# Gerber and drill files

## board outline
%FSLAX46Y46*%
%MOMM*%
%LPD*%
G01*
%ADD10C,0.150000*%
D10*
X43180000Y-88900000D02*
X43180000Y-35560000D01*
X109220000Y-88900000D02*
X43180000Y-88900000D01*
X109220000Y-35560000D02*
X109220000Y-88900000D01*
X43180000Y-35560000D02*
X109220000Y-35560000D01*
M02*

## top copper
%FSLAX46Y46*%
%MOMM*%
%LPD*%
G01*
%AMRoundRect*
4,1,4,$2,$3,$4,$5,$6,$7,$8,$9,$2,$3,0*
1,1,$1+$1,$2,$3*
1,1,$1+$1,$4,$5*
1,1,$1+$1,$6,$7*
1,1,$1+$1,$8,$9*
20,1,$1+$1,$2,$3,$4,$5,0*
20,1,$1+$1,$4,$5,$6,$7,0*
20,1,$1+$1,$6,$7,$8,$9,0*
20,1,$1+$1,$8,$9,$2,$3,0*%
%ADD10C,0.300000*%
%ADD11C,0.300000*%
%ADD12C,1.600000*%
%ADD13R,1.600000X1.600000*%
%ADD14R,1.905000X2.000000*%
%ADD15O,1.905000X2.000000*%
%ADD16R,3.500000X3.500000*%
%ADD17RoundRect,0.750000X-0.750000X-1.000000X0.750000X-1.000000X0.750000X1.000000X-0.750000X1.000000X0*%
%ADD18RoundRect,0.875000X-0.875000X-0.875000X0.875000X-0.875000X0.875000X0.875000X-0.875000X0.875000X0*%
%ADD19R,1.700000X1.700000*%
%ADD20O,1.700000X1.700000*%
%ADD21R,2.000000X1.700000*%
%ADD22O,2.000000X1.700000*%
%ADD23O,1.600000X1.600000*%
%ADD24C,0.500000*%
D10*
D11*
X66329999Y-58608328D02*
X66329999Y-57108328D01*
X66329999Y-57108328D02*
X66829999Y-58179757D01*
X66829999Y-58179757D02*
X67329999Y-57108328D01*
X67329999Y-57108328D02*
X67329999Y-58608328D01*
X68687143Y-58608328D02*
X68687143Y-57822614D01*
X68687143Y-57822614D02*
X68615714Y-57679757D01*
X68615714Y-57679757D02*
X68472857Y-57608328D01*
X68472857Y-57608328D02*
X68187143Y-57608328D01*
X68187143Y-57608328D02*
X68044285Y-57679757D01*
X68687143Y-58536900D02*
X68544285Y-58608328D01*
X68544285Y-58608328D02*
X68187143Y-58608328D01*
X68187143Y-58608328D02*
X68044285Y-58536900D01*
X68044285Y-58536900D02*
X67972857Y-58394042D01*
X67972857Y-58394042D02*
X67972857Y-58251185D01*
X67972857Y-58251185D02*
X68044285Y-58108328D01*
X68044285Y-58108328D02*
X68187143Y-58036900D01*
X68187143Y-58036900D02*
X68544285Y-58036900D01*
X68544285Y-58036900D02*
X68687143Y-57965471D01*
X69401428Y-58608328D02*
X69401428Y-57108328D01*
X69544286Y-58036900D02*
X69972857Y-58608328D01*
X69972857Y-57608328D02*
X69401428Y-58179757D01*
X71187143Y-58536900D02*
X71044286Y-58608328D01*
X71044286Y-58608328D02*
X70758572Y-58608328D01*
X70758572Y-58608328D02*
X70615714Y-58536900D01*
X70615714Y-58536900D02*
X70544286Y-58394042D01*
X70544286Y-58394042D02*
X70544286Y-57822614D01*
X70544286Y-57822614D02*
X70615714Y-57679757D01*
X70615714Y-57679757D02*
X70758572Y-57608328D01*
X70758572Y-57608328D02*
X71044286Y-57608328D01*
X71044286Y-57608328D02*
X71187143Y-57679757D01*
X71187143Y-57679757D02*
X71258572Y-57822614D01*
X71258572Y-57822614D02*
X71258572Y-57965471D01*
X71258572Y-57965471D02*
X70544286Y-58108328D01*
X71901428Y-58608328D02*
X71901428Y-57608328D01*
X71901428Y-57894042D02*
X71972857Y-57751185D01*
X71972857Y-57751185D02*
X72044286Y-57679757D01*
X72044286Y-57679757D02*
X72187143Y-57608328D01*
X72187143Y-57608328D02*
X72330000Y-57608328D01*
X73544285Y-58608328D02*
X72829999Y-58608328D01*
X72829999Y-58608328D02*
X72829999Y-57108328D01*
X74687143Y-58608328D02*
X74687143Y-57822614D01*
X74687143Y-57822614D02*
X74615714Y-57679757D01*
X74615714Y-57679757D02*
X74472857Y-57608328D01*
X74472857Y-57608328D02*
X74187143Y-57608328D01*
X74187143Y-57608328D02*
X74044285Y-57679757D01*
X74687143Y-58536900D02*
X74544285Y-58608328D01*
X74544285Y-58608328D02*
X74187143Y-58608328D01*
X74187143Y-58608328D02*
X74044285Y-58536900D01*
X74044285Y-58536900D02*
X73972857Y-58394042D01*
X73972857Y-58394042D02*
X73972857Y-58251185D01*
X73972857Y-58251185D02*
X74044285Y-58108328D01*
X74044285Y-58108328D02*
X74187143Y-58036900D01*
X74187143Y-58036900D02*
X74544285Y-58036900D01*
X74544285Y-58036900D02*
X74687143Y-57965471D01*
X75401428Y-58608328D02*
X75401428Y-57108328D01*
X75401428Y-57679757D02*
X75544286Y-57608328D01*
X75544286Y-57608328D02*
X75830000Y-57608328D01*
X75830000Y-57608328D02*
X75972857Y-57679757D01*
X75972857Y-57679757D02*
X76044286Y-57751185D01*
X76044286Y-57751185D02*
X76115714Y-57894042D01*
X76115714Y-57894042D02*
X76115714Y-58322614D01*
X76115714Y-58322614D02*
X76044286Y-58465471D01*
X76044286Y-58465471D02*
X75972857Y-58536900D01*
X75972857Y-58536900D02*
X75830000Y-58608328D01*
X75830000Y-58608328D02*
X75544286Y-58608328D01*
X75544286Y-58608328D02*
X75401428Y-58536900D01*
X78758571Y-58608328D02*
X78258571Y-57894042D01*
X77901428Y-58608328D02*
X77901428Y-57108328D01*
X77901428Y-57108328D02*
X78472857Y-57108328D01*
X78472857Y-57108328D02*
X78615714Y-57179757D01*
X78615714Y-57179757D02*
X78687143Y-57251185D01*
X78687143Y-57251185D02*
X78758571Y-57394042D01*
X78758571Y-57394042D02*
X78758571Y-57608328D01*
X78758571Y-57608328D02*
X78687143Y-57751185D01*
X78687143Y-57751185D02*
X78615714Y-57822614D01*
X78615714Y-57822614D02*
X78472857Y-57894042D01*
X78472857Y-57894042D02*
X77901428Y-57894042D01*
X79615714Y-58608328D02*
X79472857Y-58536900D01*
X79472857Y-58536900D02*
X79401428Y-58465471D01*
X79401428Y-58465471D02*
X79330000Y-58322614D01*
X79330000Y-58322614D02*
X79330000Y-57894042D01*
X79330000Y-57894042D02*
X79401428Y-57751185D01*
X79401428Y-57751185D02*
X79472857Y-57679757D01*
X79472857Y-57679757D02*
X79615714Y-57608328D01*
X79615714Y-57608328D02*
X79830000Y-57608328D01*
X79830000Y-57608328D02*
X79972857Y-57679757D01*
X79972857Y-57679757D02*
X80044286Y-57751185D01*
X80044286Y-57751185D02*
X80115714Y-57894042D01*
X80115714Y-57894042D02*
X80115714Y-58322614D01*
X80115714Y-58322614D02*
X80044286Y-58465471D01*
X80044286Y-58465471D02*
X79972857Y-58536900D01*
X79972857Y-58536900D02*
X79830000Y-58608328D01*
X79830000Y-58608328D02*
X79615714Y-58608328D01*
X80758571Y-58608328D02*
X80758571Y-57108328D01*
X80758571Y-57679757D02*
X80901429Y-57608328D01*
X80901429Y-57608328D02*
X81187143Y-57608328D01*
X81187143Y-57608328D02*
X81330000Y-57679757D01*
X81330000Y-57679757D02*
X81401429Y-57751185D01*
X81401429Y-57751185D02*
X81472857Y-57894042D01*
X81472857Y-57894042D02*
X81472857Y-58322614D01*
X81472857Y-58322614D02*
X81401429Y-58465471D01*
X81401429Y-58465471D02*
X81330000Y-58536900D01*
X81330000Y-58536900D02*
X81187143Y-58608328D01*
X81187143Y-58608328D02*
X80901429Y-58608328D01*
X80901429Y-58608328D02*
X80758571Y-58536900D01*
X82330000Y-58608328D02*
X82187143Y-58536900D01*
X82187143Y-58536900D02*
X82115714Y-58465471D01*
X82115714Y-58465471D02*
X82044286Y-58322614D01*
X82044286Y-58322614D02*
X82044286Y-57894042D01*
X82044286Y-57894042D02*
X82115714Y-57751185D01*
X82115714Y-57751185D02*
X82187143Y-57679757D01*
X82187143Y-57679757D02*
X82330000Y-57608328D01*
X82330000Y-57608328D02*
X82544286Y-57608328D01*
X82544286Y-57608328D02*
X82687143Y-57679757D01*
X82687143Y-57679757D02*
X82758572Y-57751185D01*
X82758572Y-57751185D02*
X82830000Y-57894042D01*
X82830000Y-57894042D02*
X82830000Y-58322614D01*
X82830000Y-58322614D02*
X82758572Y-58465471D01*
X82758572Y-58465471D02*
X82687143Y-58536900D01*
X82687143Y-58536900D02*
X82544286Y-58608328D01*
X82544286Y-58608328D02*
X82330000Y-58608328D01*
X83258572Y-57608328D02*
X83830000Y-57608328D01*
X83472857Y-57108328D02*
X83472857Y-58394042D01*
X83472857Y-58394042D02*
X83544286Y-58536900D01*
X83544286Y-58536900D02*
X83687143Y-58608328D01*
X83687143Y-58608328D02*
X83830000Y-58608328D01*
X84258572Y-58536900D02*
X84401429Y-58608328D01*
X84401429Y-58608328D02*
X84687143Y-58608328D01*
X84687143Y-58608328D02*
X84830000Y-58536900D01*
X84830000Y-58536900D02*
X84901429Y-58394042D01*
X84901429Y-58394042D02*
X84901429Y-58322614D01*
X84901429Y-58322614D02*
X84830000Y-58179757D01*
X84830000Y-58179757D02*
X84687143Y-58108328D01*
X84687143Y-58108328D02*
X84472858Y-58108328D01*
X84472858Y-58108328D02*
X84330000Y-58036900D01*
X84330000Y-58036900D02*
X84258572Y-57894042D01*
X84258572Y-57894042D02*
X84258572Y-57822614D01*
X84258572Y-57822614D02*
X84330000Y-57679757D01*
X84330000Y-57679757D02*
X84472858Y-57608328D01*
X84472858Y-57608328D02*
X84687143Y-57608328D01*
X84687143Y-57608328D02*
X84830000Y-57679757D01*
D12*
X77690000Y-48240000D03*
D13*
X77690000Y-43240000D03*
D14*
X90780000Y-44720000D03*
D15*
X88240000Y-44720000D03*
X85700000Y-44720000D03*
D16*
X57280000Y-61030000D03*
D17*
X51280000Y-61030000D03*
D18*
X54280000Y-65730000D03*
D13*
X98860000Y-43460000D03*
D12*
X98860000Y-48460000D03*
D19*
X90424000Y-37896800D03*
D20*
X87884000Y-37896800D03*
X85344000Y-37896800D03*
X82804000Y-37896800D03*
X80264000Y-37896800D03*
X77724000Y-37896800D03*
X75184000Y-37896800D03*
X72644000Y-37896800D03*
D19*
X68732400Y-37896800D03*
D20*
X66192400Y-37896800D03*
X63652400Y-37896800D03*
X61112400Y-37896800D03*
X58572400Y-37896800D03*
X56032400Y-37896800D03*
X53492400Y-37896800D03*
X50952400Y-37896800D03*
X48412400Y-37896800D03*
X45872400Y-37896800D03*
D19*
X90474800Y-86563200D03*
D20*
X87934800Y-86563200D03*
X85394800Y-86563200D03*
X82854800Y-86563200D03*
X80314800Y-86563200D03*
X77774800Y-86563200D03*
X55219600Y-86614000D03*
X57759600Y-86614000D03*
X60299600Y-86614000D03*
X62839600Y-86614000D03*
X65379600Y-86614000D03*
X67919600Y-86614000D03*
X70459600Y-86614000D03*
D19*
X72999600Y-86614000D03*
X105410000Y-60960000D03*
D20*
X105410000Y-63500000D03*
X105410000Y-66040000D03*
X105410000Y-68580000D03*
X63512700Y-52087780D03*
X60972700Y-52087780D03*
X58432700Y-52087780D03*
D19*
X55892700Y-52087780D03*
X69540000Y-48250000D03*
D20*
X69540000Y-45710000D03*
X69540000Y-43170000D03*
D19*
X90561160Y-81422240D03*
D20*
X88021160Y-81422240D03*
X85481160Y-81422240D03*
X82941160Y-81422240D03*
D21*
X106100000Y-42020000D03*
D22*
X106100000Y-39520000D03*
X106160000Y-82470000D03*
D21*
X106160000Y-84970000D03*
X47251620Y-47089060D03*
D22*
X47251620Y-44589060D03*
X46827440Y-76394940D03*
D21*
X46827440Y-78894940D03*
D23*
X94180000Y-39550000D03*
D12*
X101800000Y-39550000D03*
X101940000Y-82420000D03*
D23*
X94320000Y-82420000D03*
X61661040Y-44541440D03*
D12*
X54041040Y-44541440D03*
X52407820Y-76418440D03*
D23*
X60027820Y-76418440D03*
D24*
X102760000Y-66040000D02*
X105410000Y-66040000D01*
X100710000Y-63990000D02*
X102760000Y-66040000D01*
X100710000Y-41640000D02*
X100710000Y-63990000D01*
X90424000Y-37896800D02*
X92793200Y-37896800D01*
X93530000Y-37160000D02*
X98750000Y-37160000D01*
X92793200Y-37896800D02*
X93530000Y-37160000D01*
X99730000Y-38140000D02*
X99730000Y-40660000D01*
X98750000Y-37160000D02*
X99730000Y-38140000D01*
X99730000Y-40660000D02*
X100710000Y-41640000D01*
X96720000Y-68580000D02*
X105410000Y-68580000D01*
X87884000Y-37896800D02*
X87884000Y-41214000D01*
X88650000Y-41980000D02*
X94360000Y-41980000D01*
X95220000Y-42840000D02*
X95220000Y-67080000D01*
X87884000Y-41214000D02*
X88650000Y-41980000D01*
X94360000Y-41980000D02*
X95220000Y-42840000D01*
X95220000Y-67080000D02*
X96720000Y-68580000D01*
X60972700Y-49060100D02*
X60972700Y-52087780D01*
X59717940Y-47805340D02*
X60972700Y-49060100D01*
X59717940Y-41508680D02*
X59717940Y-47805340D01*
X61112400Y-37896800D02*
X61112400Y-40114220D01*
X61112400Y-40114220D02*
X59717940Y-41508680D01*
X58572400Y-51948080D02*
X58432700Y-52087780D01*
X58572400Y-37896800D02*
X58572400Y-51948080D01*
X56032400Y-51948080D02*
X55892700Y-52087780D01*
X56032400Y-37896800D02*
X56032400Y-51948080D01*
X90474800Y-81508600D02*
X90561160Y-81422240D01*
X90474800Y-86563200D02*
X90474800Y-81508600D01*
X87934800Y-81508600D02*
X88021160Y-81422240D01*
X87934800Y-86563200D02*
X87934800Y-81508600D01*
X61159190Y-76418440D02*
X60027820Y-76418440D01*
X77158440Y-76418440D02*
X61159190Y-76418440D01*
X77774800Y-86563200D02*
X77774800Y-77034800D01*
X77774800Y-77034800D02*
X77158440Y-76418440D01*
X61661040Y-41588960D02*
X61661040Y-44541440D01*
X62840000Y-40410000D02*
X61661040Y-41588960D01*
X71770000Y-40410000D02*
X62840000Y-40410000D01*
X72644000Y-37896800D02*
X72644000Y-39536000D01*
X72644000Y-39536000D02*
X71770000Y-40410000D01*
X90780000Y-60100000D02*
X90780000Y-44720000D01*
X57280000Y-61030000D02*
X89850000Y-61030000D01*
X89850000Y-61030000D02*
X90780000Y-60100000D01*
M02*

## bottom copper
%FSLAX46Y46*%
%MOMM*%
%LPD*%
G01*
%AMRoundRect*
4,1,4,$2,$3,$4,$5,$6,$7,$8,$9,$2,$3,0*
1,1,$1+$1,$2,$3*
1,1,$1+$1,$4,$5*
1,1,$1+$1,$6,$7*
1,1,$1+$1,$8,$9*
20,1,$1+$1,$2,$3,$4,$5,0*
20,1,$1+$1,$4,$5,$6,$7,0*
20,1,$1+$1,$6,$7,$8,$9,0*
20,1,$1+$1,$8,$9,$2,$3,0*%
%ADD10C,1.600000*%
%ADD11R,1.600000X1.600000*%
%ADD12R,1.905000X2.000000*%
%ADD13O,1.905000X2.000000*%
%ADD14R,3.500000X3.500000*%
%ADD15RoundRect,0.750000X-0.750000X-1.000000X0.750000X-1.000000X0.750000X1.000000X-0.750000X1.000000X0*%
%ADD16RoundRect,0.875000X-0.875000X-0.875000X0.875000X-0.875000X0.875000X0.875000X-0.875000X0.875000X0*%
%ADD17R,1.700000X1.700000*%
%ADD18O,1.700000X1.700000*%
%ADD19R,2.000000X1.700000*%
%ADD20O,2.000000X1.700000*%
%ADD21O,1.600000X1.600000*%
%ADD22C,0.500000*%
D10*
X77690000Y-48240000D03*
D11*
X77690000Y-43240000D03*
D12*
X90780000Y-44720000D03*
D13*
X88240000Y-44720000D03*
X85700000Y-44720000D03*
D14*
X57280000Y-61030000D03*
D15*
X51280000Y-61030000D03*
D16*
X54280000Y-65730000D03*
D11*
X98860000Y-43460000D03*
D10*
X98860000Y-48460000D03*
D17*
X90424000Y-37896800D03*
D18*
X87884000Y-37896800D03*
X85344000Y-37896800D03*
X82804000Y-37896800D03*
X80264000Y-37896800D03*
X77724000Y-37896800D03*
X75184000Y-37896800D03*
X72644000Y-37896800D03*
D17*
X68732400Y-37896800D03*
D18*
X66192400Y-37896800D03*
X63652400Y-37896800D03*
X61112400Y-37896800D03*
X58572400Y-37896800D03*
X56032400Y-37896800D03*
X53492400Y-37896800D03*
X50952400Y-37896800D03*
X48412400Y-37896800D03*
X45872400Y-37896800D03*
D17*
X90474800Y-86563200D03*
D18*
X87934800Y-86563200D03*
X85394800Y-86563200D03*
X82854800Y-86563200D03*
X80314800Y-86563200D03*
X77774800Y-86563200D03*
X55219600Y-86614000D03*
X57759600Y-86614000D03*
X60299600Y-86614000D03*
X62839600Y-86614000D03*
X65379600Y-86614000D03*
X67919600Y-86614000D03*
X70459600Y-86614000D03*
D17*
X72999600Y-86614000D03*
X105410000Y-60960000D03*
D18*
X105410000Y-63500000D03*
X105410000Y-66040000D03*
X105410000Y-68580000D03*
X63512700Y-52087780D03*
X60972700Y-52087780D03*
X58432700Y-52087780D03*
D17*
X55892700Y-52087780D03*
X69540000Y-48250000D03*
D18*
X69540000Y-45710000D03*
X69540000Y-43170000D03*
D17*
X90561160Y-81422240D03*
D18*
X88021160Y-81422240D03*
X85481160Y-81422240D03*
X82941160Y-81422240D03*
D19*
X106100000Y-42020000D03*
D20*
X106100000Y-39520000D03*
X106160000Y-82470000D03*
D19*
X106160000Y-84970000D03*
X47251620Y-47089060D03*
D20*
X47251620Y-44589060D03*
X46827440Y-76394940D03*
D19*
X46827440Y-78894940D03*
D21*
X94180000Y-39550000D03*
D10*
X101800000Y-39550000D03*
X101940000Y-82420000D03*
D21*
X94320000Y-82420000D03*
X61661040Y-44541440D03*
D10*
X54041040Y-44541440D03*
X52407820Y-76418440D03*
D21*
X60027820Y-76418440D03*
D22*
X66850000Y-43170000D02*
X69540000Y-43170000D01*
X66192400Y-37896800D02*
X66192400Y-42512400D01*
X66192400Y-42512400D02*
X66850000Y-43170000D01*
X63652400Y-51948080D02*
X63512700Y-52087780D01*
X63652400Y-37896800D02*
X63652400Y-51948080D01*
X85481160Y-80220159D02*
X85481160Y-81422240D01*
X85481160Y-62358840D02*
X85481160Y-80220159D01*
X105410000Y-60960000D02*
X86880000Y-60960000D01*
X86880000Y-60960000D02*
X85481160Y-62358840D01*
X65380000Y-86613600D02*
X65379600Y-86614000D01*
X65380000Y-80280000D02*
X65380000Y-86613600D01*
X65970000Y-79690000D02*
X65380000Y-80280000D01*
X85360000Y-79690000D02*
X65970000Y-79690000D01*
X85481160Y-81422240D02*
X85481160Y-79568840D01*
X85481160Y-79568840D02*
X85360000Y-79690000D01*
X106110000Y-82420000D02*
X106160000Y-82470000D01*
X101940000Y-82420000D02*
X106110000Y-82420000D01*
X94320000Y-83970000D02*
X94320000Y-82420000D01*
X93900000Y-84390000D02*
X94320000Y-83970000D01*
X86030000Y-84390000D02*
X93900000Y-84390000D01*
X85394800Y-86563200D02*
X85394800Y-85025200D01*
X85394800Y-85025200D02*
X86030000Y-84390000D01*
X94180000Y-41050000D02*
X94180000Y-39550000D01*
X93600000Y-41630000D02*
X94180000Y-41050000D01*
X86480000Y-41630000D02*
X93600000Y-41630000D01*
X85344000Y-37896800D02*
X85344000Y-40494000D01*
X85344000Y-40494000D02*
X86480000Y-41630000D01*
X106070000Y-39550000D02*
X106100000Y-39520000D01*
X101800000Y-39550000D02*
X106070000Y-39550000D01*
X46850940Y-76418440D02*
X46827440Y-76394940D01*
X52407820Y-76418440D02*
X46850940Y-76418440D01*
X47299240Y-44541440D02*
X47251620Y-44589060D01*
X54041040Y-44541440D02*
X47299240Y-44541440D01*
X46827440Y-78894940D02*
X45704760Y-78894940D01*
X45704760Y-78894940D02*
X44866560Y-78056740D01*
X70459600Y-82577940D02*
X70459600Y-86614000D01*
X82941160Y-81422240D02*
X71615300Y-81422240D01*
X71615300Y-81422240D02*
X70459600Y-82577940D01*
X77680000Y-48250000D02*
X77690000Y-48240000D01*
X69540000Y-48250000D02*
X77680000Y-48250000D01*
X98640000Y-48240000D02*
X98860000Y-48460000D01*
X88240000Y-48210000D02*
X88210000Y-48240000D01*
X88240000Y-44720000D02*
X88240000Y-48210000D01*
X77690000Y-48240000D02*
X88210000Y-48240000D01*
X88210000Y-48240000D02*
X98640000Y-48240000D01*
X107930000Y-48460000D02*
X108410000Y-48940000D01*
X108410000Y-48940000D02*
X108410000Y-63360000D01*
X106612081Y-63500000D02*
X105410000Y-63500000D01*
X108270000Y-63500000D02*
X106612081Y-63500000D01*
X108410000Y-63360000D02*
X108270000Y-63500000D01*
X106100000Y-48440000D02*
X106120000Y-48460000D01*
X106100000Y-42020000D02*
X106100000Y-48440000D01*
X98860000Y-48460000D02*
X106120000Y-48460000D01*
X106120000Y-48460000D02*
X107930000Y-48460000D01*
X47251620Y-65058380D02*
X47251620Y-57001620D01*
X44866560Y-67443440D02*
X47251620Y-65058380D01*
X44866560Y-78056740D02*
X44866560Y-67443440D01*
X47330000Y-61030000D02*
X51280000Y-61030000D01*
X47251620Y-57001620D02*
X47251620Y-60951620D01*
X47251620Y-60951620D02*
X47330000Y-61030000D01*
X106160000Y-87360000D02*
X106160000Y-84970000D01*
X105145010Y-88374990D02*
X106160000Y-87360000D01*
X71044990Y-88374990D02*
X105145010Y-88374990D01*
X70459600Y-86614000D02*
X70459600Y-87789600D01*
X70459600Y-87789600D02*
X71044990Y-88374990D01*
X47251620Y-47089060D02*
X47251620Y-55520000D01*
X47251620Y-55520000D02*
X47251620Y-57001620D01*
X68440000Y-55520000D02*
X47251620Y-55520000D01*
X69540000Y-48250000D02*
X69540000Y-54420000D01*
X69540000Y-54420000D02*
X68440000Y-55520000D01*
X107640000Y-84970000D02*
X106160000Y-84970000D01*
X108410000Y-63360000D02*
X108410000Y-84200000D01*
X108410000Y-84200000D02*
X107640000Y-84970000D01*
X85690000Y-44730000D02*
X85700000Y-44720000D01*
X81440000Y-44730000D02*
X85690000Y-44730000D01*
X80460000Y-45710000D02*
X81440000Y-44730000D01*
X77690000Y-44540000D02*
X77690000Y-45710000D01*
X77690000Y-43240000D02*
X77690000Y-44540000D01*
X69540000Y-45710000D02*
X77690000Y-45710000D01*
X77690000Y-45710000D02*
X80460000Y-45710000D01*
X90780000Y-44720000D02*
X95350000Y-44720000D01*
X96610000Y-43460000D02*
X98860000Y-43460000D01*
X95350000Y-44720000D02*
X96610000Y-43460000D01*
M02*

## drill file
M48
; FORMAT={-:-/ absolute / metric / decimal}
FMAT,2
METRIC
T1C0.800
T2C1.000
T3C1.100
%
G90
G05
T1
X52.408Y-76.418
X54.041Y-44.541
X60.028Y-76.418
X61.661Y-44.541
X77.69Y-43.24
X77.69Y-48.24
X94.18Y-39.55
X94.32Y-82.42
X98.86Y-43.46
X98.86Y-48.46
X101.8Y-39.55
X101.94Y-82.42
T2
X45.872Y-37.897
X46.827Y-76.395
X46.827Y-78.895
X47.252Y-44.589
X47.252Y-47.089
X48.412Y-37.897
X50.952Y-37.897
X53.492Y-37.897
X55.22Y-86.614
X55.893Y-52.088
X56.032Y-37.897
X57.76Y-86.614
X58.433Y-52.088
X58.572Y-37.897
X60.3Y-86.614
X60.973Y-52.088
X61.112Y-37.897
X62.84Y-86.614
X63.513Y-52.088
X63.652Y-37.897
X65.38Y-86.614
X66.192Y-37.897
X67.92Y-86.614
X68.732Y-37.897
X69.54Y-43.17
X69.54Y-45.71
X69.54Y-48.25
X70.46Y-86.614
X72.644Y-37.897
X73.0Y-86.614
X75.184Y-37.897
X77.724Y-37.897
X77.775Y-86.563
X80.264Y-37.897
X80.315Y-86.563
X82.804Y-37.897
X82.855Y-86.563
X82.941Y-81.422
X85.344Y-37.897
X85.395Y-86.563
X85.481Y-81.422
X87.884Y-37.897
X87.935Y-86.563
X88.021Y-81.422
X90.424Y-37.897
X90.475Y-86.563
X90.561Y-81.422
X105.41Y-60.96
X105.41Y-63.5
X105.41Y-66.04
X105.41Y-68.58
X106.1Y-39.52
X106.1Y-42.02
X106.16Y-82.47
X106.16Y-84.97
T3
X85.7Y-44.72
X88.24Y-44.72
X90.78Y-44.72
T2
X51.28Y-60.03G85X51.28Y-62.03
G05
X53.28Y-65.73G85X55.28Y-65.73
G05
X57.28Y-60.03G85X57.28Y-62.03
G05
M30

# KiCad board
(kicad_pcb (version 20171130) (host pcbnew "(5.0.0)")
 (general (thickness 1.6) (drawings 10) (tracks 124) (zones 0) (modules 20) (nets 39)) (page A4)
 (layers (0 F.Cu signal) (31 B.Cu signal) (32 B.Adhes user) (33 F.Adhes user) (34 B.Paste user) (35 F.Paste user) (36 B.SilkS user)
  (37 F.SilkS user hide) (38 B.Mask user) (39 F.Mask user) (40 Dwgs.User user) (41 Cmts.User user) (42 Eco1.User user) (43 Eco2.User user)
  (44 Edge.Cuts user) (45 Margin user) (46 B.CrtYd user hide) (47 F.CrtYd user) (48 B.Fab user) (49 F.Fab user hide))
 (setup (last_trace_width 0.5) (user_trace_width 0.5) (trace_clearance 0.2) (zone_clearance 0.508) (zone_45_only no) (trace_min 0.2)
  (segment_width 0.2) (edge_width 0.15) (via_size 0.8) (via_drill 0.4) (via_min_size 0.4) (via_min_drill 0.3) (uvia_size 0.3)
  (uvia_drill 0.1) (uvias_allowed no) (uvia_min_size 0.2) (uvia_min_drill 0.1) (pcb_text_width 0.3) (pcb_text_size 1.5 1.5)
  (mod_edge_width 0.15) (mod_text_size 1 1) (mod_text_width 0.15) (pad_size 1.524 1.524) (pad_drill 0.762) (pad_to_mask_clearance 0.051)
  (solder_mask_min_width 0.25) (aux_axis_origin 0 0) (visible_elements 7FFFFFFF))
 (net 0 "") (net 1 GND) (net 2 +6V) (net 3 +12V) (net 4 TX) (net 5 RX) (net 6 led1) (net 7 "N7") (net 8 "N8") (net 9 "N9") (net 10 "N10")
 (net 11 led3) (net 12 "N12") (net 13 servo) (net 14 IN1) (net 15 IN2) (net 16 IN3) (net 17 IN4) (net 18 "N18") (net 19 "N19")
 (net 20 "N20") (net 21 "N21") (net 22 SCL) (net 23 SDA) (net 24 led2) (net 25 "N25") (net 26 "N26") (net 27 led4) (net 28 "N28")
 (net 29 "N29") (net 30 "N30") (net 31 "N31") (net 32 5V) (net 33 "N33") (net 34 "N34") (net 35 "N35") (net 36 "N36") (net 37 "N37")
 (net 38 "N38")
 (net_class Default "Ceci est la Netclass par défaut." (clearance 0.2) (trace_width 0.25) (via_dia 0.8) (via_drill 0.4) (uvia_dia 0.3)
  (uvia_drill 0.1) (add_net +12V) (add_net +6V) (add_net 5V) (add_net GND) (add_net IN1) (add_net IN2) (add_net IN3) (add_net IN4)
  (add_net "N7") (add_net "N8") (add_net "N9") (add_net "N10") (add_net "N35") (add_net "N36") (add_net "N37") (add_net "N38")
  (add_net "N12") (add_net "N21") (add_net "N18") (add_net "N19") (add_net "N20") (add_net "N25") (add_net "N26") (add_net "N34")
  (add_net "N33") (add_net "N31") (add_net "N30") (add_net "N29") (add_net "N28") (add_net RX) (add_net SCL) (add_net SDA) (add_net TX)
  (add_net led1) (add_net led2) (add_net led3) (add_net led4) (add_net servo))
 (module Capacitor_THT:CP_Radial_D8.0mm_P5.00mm (layer F.Cu) (at 77.69 43.24 270)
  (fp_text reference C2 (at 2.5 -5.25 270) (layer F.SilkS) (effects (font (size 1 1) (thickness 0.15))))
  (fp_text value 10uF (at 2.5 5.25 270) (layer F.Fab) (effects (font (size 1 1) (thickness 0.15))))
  (pad 2 thru_hole circle (at 5 0 270) (size 1.6 1.6) (drill 0.8) (layers *.Cu *.Mask) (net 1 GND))
  (pad 1 thru_hole rect (at 0 0 270) (size 1.6 1.6) (drill 0.8) (layers *.Cu *.Mask) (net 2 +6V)))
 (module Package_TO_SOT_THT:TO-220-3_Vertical (layer F.Cu) (at 90.78 44.72 180)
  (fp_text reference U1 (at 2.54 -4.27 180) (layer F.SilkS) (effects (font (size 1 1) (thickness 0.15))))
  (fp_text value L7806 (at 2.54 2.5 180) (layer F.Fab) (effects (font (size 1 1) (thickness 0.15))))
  (pad 1 thru_hole rect (at 0 0 180) (size 1.905 2) (drill 1.1) (layers *.Cu *.Mask) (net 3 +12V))
  (pad 2 thru_hole oval (at 2.54 0 180) (size 1.905 2) (drill 1.1) (layers *.Cu *.Mask) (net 1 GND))
  (pad 3 thru_hole oval (at 5.08 0 180) (size 1.905 2) (drill 1.1) (layers *.Cu *.Mask) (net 2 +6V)))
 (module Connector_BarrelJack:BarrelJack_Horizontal (layer F.Cu) (at 57.28 61.03)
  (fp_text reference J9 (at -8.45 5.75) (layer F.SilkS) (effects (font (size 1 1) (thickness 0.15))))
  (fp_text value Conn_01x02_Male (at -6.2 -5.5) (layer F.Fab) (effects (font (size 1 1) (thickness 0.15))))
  (pad 1 thru_hole rect (at 0 0) (size 3.5 3.5) (drill oval 1 3) (layers *.Cu *.Mask) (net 3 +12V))
  (pad 2 thru_hole roundrect (at -6 0) (size 3 3.5) (drill oval 1 3) (layers *.Cu *.Mask) (roundrect_rratio 0.25) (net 1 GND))
  (pad 3 thru_hole roundrect (at -3 4.7) (size 3.5 3.5) (drill oval 3 1) (layers *.Cu *.Mask) (roundrect_rratio 0.25)))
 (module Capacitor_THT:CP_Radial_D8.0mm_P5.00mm (layer F.Cu) (at 98.86 43.46 270)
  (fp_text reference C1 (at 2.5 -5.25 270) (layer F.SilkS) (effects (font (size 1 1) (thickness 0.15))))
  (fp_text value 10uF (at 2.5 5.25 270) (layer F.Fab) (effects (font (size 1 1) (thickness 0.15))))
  (pad 1 thru_hole rect (at 0 0 270) (size 1.6 1.6) (drill 0.8) (layers *.Cu *.Mask) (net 3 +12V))
  (pad 2 thru_hole circle (at 5 0 270) (size 1.6 1.6) (drill 0.8) (layers *.Cu *.Mask) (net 1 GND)))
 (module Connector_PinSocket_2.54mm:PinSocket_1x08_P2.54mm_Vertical (layer F.Cu) (at 90.424 37.8968 270)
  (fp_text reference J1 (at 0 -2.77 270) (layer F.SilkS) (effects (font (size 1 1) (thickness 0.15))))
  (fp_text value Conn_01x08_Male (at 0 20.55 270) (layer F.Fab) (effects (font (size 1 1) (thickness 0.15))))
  (pad 1 thru_hole rect (at 0 0 270) (size 1.7 1.7) (drill 1) (layers *.Cu *.Mask) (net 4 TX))
  (pad 2 thru_hole oval (at 0 2.54 270) (size 1.7 1.7) (drill 1) (layers *.Cu *.Mask) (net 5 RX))
  (pad 3 thru_hole oval (at 0 5.08 270) (size 1.7 1.7) (drill 1) (layers *.Cu *.Mask) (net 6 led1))
  (pad 4 thru_hole oval (at 0 7.62 270) (size 1.7 1.7) (drill 1) (layers *.Cu *.Mask) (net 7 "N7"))
  (pad 5 thru_hole oval (at 0 10.16 270) (size 1.7 1.7) (drill 1) (layers *.Cu *.Mask) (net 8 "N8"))
  (pad 6 thru_hole oval (at 0 12.7 270) (size 1.7 1.7) (drill 1) (layers *.Cu *.Mask) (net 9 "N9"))
  (pad 7 thru_hole oval (at 0 15.24 270) (size 1.7 1.7) (drill 1) (layers *.Cu *.Mask) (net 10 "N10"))
  (pad 8 thru_hole oval (at 0 17.78 270) (size 1.7 1.7) (drill 1) (layers *.Cu *.Mask) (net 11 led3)))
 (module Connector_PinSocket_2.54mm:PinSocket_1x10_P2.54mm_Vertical (layer F.Cu) (at 68.7324 37.8968 270)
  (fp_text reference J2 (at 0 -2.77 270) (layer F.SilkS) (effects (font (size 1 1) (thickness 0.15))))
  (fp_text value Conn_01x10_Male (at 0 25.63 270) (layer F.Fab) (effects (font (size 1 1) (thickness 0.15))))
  (pad 1 thru_hole rect (at 0 0 270) (size 1.7 1.7) (drill 1) (layers *.Cu *.Mask) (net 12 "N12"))
  (pad 2 thru_hole oval (at 0 2.54 270) (size 1.7 1.7) (drill 1) (layers *.Cu *.Mask) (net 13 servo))
  (pad 3 thru_hole oval (at 0 5.08 270) (size 1.7 1.7) (drill 1) (layers *.Cu *.Mask) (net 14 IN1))
  (pad 4 thru_hole oval (at 0 7.62 270) (size 1.7 1.7) (drill 1) (layers *.Cu *.Mask) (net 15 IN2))
  (pad 5 thru_hole oval (at 0 10.16 270) (size 1.7 1.7) (drill 1) (layers *.Cu *.Mask) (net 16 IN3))
  (pad 6 thru_hole oval (at 0 12.7 270) (size 1.7 1.7) (drill 1) (layers *.Cu *.Mask) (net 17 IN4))
  (pad 7 thru_hole oval (at 0 15.24 270) (size 1.7 1.7) (drill 1) (layers *.Cu *.Mask) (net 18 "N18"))
  (pad 8 thru_hole oval (at 0 17.78 270) (size 1.7 1.7) (drill 1) (layers *.Cu *.Mask) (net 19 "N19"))
  (pad 9 thru_hole oval (at 0 20.32 270) (size 1.7 1.7) (drill 1) (layers *.Cu *.Mask) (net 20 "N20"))
  (pad 10 thru_hole oval (at 0 22.86 270) (size 1.7 1.7) (drill 1) (layers *.Cu *.Mask) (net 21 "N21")))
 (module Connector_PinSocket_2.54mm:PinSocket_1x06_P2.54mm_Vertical (layer F.Cu) (at 90.4748 86.5632 270)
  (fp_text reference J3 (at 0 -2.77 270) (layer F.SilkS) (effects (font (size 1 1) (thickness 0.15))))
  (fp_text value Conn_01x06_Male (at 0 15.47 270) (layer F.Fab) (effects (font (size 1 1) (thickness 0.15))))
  (pad 1 thru_hole rect (at 0 0 270) (size 1.7 1.7) (drill 1) (layers *.Cu *.Mask) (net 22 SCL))
  (pad 2 thru_hole oval (at 0 2.54 270) (size 1.7 1.7) (drill 1) (layers *.Cu *.Mask) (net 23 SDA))
  (pad 3 thru_hole oval (at 0 5.08 270) (size 1.7 1.7) (drill 1) (layers *.Cu *.Mask) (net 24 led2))
  (pad 4 thru_hole oval (at 0 7.62 270) (size 1.7 1.7) (drill 1) (layers *.Cu *.Mask) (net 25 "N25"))
  (pad 5 thru_hole oval (at 0 10.16 270) (size 1.7 1.7) (drill 1) (layers *.Cu *.Mask) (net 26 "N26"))
  (pad 6 thru_hole oval (at 0 12.7 270) (size 1.7 1.7) (drill 1) (layers *.Cu *.Mask) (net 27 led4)))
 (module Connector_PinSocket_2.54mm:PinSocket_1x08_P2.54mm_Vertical (layer F.Cu) (at 72.9996 86.614 270)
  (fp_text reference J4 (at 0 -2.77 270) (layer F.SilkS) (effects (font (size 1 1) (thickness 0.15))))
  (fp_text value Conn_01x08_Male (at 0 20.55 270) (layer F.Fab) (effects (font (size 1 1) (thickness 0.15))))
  (pad 8 thru_hole oval (at 0 17.78 270) (size 1.7 1.7) (drill 1) (layers *.Cu *.Mask) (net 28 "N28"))
  (pad 7 thru_hole oval (at 0 15.24 270) (size 1.7 1.7) (drill 1) (layers *.Cu *.Mask) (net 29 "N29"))
  (pad 6 thru_hole oval (at 0 12.7 270) (size 1.7 1.7) (drill 1) (layers *.Cu *.Mask) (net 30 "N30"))
  (pad 5 thru_hole oval (at 0 10.16 270) (size 1.7 1.7) (drill 1) (layers *.Cu *.Mask) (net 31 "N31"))
  (pad 4 thru_hole oval (at 0 7.62 270) (size 1.7 1.7) (drill 1) (layers *.Cu *.Mask) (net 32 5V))
  (pad 3 thru_hole oval (at 0 5.08 270) (size 1.7 1.7) (drill 1) (layers *.Cu *.Mask) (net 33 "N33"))
  (pad 2 thru_hole oval (at 0 2.54 270) (size 1.7 1.7) (drill 1) (layers *.Cu *.Mask) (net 1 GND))
  (pad 1 thru_hole rect (at 0 0 270) (size 1.7 1.7) (drill 1) (layers *.Cu *.Mask) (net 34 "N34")))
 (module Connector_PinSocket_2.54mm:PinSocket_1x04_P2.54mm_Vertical (layer F.Cu) (at 105.41 60.96)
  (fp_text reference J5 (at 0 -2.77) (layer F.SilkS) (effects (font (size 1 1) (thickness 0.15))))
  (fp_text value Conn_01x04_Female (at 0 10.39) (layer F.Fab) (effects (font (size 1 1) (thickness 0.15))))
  (pad 1 thru_hole rect (at 0 0) (size 1.7 1.7) (drill 1) (layers *.Cu *.Mask) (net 32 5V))
  (pad 2 thru_hole oval (at 0 2.54) (size 1.7 1.7) (drill 1) (layers *.Cu *.Mask) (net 1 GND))
  (pad 3 thru_hole oval (at 0 5.08) (size 1.7 1.7) (drill 1) (layers *.Cu *.Mask) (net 4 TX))
  (pad 4 thru_hole oval (at 0 7.62) (size 1.7 1.7) (drill 1) (layers *.Cu *.Mask) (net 5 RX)))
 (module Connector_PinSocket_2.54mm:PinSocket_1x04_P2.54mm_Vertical (layer F.Cu) (at 55.8927 52.08778 90)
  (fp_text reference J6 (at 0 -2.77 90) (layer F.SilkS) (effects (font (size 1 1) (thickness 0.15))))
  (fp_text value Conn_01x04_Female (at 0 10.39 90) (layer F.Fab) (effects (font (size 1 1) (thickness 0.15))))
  (pad 4 thru_hole oval (at 0 7.62 90) (size 1.7 1.7) (drill 1) (layers *.Cu *.Mask) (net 14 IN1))
  (pad 3 thru_hole oval (at 0 5.08 90) (size 1.7 1.7) (drill 1) (layers *.Cu *.Mask) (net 15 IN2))
  (pad 2 thru_hole oval (at 0 2.54 90) (size 1.7 1.7) (drill 1) (layers *.Cu *.Mask) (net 16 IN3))
  (pad 1 thru_hole rect (at 0 0 90) (size 1.7 1.7) (drill 1) (layers *.Cu *.Mask) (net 17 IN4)))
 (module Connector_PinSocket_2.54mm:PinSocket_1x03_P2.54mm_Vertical (layer F.Cu) (at 69.54 48.25 180)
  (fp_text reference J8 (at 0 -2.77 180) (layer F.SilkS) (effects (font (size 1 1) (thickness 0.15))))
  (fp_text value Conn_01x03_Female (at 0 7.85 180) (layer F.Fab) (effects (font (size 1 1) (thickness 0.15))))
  (pad 1 thru_hole rect (at 0 0 180) (size 1.7 1.7) (drill 1) (layers *.Cu *.Mask) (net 1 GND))
  (pad 2 thru_hole oval (at 0 2.54 180) (size 1.7 1.7) (drill 1) (layers *.Cu *.Mask) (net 2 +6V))
  (pad 3 thru_hole oval (at 0 5.08 180) (size 1.7 1.7) (drill 1) (layers *.Cu *.Mask) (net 13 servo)))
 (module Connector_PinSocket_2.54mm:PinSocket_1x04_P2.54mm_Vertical (layer F.Cu) (at 90.56116 81.42224 270)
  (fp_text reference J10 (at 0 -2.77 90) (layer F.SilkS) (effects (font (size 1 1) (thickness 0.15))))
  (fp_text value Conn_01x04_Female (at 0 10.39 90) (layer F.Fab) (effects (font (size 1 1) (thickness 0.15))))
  (pad 1 thru_hole rect (at 0 0 270) (size 1.7 1.7) (drill 1) (layers *.Cu *.Mask) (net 22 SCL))
  (pad 2 thru_hole oval (at 0 2.54 270) (size 1.7 1.7) (drill 1) (layers *.Cu *.Mask) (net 23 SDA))
  (pad 3 thru_hole oval (at 0 5.08 270) (size 1.7 1.7) (drill 1) (layers *.Cu *.Mask) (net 32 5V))
  (pad 4 thru_hole oval (at 0 7.62 270) (size 1.7 1.7) (drill 1) (layers *.Cu *.Mask) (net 1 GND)))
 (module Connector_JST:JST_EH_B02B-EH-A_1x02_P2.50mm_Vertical (layer F.Cu) (at 106.1 42.02 90)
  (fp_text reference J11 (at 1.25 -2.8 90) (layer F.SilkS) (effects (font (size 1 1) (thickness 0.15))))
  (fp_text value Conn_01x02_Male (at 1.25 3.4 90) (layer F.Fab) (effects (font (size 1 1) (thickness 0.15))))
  (pad 1 thru_hole rect (at 0 0 90) (size 1.7 2) (drill 1) (layers *.Cu *.Mask) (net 1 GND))
  (pad 2 thru_hole oval (at 2.5 0 90) (size 1.7 2) (drill 1) (layers *.Cu *.Mask) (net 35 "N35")))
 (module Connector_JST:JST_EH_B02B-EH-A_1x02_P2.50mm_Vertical (layer F.Cu) (at 106.16 84.97 90)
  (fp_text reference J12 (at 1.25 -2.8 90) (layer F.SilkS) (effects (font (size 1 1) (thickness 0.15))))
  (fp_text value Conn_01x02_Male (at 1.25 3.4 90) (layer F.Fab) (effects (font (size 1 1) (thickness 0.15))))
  (pad 2 thru_hole oval (at 2.5 0 90) (size 1.7 2) (drill 1) (layers *.Cu *.Mask) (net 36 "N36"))
  (pad 1 thru_hole rect (at 0 0 90) (size 1.7 2) (drill 1) (layers *.Cu *.Mask) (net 1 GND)))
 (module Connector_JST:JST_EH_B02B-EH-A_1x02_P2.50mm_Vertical (layer F.Cu) (at 47.25162 47.08906 90)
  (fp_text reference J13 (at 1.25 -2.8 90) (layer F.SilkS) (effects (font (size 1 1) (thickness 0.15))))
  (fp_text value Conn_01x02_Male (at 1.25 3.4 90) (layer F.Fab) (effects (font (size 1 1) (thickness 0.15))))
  (pad 1 thru_hole rect (at 0 0 90) (size 1.7 2) (drill 1) (layers *.Cu *.Mask) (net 1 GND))
  (pad 2 thru_hole oval (at 2.5 0 90) (size 1.7 2) (drill 1) (layers *.Cu *.Mask) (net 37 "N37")))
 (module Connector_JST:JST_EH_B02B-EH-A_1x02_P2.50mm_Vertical (layer F.Cu) (at 46.82744 78.89494 90)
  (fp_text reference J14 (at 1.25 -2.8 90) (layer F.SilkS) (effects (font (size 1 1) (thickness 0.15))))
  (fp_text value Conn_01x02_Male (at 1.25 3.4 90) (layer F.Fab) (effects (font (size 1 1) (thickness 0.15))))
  (pad 2 thru_hole oval (at 2.5 0 90) (size 1.7 2) (drill 1) (layers *.Cu *.Mask) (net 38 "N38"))
  (pad 1 thru_hole rect (at 0 0 90) (size 1.7 2) (drill 1) (layers *.Cu *.Mask) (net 1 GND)))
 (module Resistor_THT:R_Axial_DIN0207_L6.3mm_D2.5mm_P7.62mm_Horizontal (layer F.Cu) (at 101.8 39.55 180)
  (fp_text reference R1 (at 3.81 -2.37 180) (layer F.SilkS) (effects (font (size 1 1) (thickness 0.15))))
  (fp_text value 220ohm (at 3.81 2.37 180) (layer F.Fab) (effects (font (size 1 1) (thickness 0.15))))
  (pad 2 thru_hole oval (at 7.62 0 180) (size 1.6 1.6) (drill 0.8) (layers *.Cu *.Mask) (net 6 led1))
  (pad 1 thru_hole circle (at 0 0 180) (size 1.6 1.6) (drill 0.8) (layers *.Cu *.Mask) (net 35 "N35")))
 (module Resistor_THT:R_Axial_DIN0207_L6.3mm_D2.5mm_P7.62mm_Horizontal (layer F.Cu) (at 101.94 82.42 180)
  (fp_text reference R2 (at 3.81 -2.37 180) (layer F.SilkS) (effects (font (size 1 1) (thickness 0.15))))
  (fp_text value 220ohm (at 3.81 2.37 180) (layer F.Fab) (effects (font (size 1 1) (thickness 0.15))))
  (pad 1 thru_hole circle (at 0 0 180) (size 1.6 1.6) (drill 0.8) (layers *.Cu *.Mask) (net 36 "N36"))
  (pad 2 thru_hole oval (at 7.62 0 180) (size 1.6 1.6) (drill 0.8) (layers *.Cu *.Mask) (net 24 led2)))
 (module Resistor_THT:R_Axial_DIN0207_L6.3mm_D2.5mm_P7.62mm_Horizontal (layer F.Cu) (at 54.04104 44.54144)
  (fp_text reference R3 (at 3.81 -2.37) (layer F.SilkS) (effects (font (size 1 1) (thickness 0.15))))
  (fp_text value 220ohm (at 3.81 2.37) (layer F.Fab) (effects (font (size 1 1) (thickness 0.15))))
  (pad 2 thru_hole oval (at 7.62 0) (size 1.6 1.6) (drill 0.8) (layers *.Cu *.Mask) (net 11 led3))
  (pad 1 thru_hole circle (at 0 0) (size 1.6 1.6) (drill 0.8) (layers *.Cu *.Mask) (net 37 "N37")))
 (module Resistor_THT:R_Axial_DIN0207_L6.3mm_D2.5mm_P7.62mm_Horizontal (layer F.Cu) (at 52.40782 76.41844)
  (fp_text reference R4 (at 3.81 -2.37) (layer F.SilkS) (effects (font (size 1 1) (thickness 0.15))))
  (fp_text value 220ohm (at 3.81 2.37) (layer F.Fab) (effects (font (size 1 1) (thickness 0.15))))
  (pad 1 thru_hole circle (at 0 0) (size 1.6 1.6) (drill 0.8) (layers *.Cu *.Mask) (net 38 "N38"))
  (pad 2 thru_hole oval (at 7.62 0) (size 1.6 1.6) (drill 0.8) (layers *.Cu *.Mask) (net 27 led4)))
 (gr_line (start 43.18 88.9) (end 43.18 35.56) (layer Edge.Cuts) (width 0.15))
 (gr_line (start 109.22 88.9) (end 43.18 88.9) (layer Edge.Cuts) (width 0.15))
 (gr_line (start 109.22 35.56) (end 109.22 88.9) (layer Edge.Cuts) (width 0.15))
 (gr_line (start 43.18 35.56) (end 109.22 35.56) (layer Edge.Cuts) (width 0.15))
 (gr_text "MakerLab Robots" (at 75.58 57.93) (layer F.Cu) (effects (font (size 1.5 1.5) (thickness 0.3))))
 (segment (start 102.76 66.04) (end 105.41 66.04) (width 0.5) (layer F.Cu) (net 4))
 (segment (start 100.71 63.99) (end 102.76 66.04) (width 0.5) (layer F.Cu) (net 4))
 (segment (start 100.71 41.64) (end 100.71 63.99) (width 0.5) (layer F.Cu) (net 4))
 (segment (start 90.424 37.8968) (end 92.7932 37.8968) (width 0.5) (layer F.Cu) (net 4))
 (segment (start 93.53 37.16) (end 98.75 37.16) (width 0.5) (layer F.Cu) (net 4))
 (segment (start 92.7932 37.8968) (end 93.53 37.16) (width 0.5) (layer F.Cu) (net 4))
 (segment (start 99.73 38.14) (end 99.73 40.66) (width 0.5) (layer F.Cu) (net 4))
 (segment (start 98.75 37.16) (end 99.73 38.14) (width 0.5) (layer F.Cu) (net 4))
 (segment (start 99.73 40.66) (end 100.71 41.64) (width 0.5) (layer F.Cu) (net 4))
 (segment (start 96.72 68.58) (end 105.41 68.58) (width 0.5) (layer F.Cu) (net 5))
 (segment (start 87.884 37.8968) (end 87.884 41.214) (width 0.5) (layer F.Cu) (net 5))
 (segment (start 88.65 41.98) (end 94.36 41.98) (width 0.5) (layer F.Cu) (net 5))
 (segment (start 95.22 42.84) (end 95.22 67.08) (width 0.5) (layer F.Cu) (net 5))
 (segment (start 87.884 41.214) (end 88.65 41.98) (width 0.5) (layer F.Cu) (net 5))
 (segment (start 94.36 41.98) (end 95.22 42.84) (width 0.5) (layer F.Cu) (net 5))
 (segment (start 95.22 67.08) (end 96.72 68.58) (width 0.5) (layer F.Cu) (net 5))
 (segment (start 66.85 43.17) (end 69.54 43.17) (width 0.5) (layer B.Cu) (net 13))
 (segment (start 66.1924 37.8968) (end 66.1924 42.5124) (width 0.5) (layer B.Cu) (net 13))
 (segment (start 66.1924 42.5124) (end 66.85 43.17) (width 0.5) (layer B.Cu) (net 13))
 (segment (start 63.6524 51.94808) (end 63.5127 52.08778) (width 0.5) (layer B.Cu) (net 14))
 (segment (start 63.6524 37.8968) (end 63.6524 51.94808) (width 0.5) (layer B.Cu) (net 14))
 (segment (start 60.9727 49.0601) (end 60.9727 52.08778) (width 0.5) (layer F.Cu) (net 15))
 (segment (start 59.71794 47.80534) (end 60.9727 49.0601) (width 0.5) (layer F.Cu) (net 15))
 (segment (start 59.71794 41.50868) (end 59.71794 47.80534) (width 0.5) (layer F.Cu) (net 15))
 (segment (start 61.1124 37.8968) (end 61.1124 40.11422) (width 0.5) (layer F.Cu) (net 15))
 (segment (start 61.1124 40.11422) (end 59.71794 41.50868) (width 0.5) (layer F.Cu) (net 15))
 (segment (start 58.5724 51.94808) (end 58.4327 52.08778) (width 0.5) (layer F.Cu) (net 16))
 (segment (start 58.5724 37.8968) (end 58.5724 51.94808) (width 0.5) (layer F.Cu) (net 16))
 (segment (start 56.0324 51.94808) (end 55.8927 52.08778) (width 0.5) (layer F.Cu) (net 17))
 (segment (start 56.0324 37.8968) (end 56.0324 51.94808) (width 0.5) (layer F.Cu) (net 17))
 (segment (start 90.4748 81.5086) (end 90.56116 81.42224) (width 0.5) (layer F.Cu) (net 22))
 (segment (start 90.4748 86.5632) (end 90.4748 81.5086) (width 0.5) (layer F.Cu) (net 22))
 (segment (start 87.9348 81.5086) (end 88.02116 81.42224) (width 0.5) (layer F.Cu) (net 23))
 (segment (start 87.9348 86.5632) (end 87.9348 81.5086) (width 0.5) (layer F.Cu) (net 23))
 (segment (start 85.48116 80.220159) (end 85.48116 81.42224) (width 0.5) (layer B.Cu) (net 32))
 (segment (start 85.48116 62.35884) (end 85.48116 80.220159) (width 0.5) (layer B.Cu) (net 32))
 (segment (start 105.41 60.96) (end 86.88 60.96) (width 0.5) (layer B.Cu) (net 32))
 (segment (start 86.88 60.96) (end 85.48116 62.35884) (width 0.5) (layer B.Cu) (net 32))
 (segment (start 65.38 86.6136) (end 65.3796 86.614) (width 0.5) (layer B.Cu) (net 32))
 (segment (start 65.38 80.28) (end 65.38 86.6136) (width 0.5) (layer B.Cu) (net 32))
 (segment (start 65.97 79.69) (end 65.38 80.28) (width 0.5) (layer B.Cu) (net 32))
 (segment (start 85.36 79.69) (end 65.97 79.69) (width 0.5) (layer B.Cu) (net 32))
 (segment (start 85.48116 81.42224) (end 85.48116 79.56884) (width 0.5) (layer B.Cu) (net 32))
 (segment (start 85.48116 79.56884) (end 85.36 79.69) (width 0.5) (layer B.Cu) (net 32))
 (segment (start 106.11 82.42) (end 106.16 82.47) (width 0.5) (layer B.Cu) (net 36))
 (segment (start 101.94 82.42) (end 106.11 82.42) (width 0.5) (layer B.Cu) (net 36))
 (segment (start 94.32 83.97) (end 94.32 82.42) (width 0.5) (layer B.Cu) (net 24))
 (segment (start 93.9 84.39) (end 94.32 83.97) (width 0.5) (layer B.Cu) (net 24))
 (segment (start 86.03 84.39) (end 93.9 84.39) (width 0.5) (layer B.Cu) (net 24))
 (segment (start 85.3948 86.5632) (end 85.3948 85.0252) (width 0.5) (layer B.Cu) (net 24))
 (segment (start 85.3948 85.0252) (end 86.03 84.39) (width 0.5) (layer B.Cu) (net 24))
 (segment (start 94.18 41.05) (end 94.18 39.55) (width 0.5) (layer B.Cu) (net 6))
 (segment (start 93.6 41.63) (end 94.18 41.05) (width 0.5) (layer B.Cu) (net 6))
 (segment (start 86.48 41.63) (end 93.6 41.63) (width 0.5) (layer B.Cu) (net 6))
 (segment (start 85.344 37.8968) (end 85.344 40.494) (width 0.5) (layer B.Cu) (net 6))
 (segment (start 85.344 40.494) (end 86.48 41.63) (width 0.5) (layer B.Cu) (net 6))
 (segment (start 106.07 39.55) (end 106.1 39.52) (width 0.5) (layer B.Cu) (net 35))
 (segment (start 101.8 39.55) (end 106.07 39.55) (width 0.5) (layer B.Cu) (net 35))
 (segment (start 46.85094 76.41844) (end 46.82744 76.39494) (width 0.5) (layer B.Cu) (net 38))
 (segment (start 52.40782 76.41844) (end 46.85094 76.41844) (width 0.5) (layer B.Cu) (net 38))
 (segment (start 61.15919 76.41844) (end 60.02782 76.41844) (width 0.5) (layer F.Cu) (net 27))
 (segment (start 77.15844 76.41844) (end 61.15919 76.41844) (width 0.5) (layer F.Cu) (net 27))
 (segment (start 77.7748 86.5632) (end 77.7748 77.0348) (width 0.5) (layer F.Cu) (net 27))
 (segment (start 77.7748 77.0348) (end 77.15844 76.41844) (width 0.5) (layer F.Cu) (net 27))
 (segment (start 61.66104 41.58896) (end 61.66104 44.54144) (width 0.5) (layer F.Cu) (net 11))
 (segment (start 62.84 40.41) (end 61.66104 41.58896) (width 0.5) (layer F.Cu) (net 11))
 (segment (start 71.77 40.41) (end 62.84 40.41) (width 0.5) (layer F.Cu) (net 11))
 (segment (start 72.644 37.8968) (end 72.644 39.536) (width 0.5) (layer F.Cu) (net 11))
 (segment (start 72.644 39.536) (end 71.77 40.41) (width 0.5) (layer F.Cu) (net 11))
 (segment (start 47.29924 44.54144) (end 47.25162 44.58906) (width 0.5) (layer B.Cu) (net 37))
 (segment (start 54.04104 44.54144) (end 47.29924 44.54144) (width 0.5) (layer B.Cu) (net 37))
 (segment (start 46.82744 78.89494) (end 45.70476 78.89494) (width 0.5) (layer B.Cu) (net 1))
 (segment (start 45.70476 78.89494) (end 44.86656 78.05674) (width 0.5) (layer B.Cu) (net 1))
 (segment (start 70.4596 82.57794) (end 70.4596 86.614) (width 0.5) (layer B.Cu) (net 1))
 (segment (start 82.94116 81.42224) (end 71.6153 81.42224) (width 0.5) (layer B.Cu) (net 1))
 (segment (start 71.6153 81.42224) (end 70.4596 82.57794) (width 0.5) (layer B.Cu) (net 1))
 (segment (start 77.68 48.25) (end 77.69 48.24) (width 0.5) (layer B.Cu) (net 1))
 (segment (start 69.54 48.25) (end 77.68 48.25) (width 0.5) (layer B.Cu) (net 1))
 (segment (start 98.64 48.24) (end 98.86 48.46) (width 0.5) (layer B.Cu) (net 1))
 (segment (start 88.24 48.21) (end 88.21 48.24) (width 0.5) (layer B.Cu) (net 1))
 (segment (start 88.24 44.72) (end 88.24 48.21) (width 0.5) (layer B.Cu) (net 1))
 (segment (start 77.69 48.24) (end 88.21 48.24) (width 0.5) (layer B.Cu) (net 1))
 (segment (start 88.21 48.24) (end 98.64 48.24) (width 0.5) (layer B.Cu) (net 1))
 (segment (start 107.93 48.46) (end 108.41 48.94) (width 0.5) (layer B.Cu) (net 1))
 (segment (start 108.41 48.94) (end 108.41 63.36) (width 0.5) (layer B.Cu) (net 1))
 (segment (start 106.612081 63.5) (end 105.41 63.5) (width 0.5) (layer B.Cu) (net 1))
 (segment (start 108.27 63.5) (end 106.612081 63.5) (width 0.5) (layer B.Cu) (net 1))
 (segment (start 108.41 63.36) (end 108.27 63.5) (width 0.5) (layer B.Cu) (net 1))
 (segment (start 106.1 48.44) (end 106.12 48.46) (width 0.5) (layer B.Cu) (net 1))
 (segment (start 106.1 42.02) (end 106.1 48.44) (width 0.5) (layer B.Cu) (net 1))
 (segment (start 98.86 48.46) (end 106.12 48.46) (width 0.5) (layer B.Cu) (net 1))
 (segment (start 106.12 48.46) (end 107.93 48.46) (width 0.5) (layer B.Cu) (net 1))
 (segment (start 47.25162 65.05838) (end 47.25162 57.00162) (width 0.5) (layer B.Cu) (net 1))
 (segment (start 44.86656 67.44344) (end 47.25162 65.05838) (width 0.5) (layer B.Cu) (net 1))
 (segment (start 44.86656 78.05674) (end 44.86656 67.44344) (width 0.5) (layer B.Cu) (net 1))
 (segment (start 47.33 61.03) (end 51.28 61.03) (width 0.5) (layer B.Cu) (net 1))
 (segment (start 47.25162 57.00162) (end 47.25162 60.95162) (width 0.5) (layer B.Cu) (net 1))
 (segment (start 47.25162 60.95162) (end 47.33 61.03) (width 0.5) (layer B.Cu) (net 1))
 (segment (start 106.16 87.36) (end 106.16 84.97) (width 0.5) (layer B.Cu) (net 1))
 (segment (start 105.14501 88.37499) (end 106.16 87.36) (width 0.5) (layer B.Cu) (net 1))
 (segment (start 71.04499 88.37499) (end 105.14501 88.37499) (width 0.5) (layer B.Cu) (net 1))
 (segment (start 70.4596 86.614) (end 70.4596 87.7896) (width 0.5) (layer B.Cu) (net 1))
 (segment (start 70.4596 87.7896) (end 71.04499 88.37499) (width 0.5) (layer B.Cu) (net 1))
 (segment (start 47.25162 47.08906) (end 47.25162 55.52) (width 0.5) (layer B.Cu) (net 1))
 (segment (start 47.25162 55.52) (end 47.25162 57.00162) (width 0.5) (layer B.Cu) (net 1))
 (segment (start 68.44 55.52) (end 47.25162 55.52) (width 0.5) (layer B.Cu) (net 1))
 (segment (start 69.54 48.25) (end 69.54 54.42) (width 0.5) (layer B.Cu) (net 1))
 (segment (start 69.54 54.42) (end 68.44 55.52) (width 0.5) (layer B.Cu) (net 1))
 (segment (start 107.64 84.97) (end 106.16 84.97) (width 0.5) (layer B.Cu) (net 1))
 (segment (start 108.41 63.36) (end 108.41 84.2) (width 0.5) (layer B.Cu) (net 1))
 (segment (start 108.41 84.2) (end 107.64 84.97) (width 0.5) (layer B.Cu) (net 1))
 (segment (start 85.69 44.73) (end 85.7 44.72) (width 0.5) (layer B.Cu) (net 2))
 (segment (start 81.44 44.73) (end 85.69 44.73) (width 0.5) (layer B.Cu) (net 2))
 (segment (start 80.46 45.71) (end 81.44 44.73) (width 0.5) (layer B.Cu) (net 2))
 (segment (start 77.69 44.54) (end 77.69 45.71) (width 0.5) (layer B.Cu) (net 2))
 (segment (start 77.69 43.24) (end 77.69 44.54) (width 0.5) (layer B.Cu) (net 2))
 (segment (start 69.54 45.71) (end 77.69 45.71) (width 0.5) (layer B.Cu) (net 2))
 (segment (start 77.69 45.71) (end 80.46 45.71) (width 0.5) (layer B.Cu) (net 2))
 (segment (start 90.78 44.72) (end 95.35 44.72) (width 0.5) (layer B.Cu) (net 3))
 (segment (start 96.61 43.46) (end 98.86 43.46) (width 0.5) (layer B.Cu) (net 3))
 (segment (start 95.35 44.72) (end 96.61 43.46) (width 0.5) (layer B.Cu) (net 3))
 (segment (start 90.78 60.1) (end 90.78 44.72) (width 0.5) (layer F.Cu) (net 3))
 (segment (start 57.28 61.03) (end 89.85 61.03) (width 0.5) (layer F.Cu) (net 3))
 (segment (start 89.85 61.03) (end 90.78 60.1) (width 0.5) (layer F.Cu) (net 3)))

